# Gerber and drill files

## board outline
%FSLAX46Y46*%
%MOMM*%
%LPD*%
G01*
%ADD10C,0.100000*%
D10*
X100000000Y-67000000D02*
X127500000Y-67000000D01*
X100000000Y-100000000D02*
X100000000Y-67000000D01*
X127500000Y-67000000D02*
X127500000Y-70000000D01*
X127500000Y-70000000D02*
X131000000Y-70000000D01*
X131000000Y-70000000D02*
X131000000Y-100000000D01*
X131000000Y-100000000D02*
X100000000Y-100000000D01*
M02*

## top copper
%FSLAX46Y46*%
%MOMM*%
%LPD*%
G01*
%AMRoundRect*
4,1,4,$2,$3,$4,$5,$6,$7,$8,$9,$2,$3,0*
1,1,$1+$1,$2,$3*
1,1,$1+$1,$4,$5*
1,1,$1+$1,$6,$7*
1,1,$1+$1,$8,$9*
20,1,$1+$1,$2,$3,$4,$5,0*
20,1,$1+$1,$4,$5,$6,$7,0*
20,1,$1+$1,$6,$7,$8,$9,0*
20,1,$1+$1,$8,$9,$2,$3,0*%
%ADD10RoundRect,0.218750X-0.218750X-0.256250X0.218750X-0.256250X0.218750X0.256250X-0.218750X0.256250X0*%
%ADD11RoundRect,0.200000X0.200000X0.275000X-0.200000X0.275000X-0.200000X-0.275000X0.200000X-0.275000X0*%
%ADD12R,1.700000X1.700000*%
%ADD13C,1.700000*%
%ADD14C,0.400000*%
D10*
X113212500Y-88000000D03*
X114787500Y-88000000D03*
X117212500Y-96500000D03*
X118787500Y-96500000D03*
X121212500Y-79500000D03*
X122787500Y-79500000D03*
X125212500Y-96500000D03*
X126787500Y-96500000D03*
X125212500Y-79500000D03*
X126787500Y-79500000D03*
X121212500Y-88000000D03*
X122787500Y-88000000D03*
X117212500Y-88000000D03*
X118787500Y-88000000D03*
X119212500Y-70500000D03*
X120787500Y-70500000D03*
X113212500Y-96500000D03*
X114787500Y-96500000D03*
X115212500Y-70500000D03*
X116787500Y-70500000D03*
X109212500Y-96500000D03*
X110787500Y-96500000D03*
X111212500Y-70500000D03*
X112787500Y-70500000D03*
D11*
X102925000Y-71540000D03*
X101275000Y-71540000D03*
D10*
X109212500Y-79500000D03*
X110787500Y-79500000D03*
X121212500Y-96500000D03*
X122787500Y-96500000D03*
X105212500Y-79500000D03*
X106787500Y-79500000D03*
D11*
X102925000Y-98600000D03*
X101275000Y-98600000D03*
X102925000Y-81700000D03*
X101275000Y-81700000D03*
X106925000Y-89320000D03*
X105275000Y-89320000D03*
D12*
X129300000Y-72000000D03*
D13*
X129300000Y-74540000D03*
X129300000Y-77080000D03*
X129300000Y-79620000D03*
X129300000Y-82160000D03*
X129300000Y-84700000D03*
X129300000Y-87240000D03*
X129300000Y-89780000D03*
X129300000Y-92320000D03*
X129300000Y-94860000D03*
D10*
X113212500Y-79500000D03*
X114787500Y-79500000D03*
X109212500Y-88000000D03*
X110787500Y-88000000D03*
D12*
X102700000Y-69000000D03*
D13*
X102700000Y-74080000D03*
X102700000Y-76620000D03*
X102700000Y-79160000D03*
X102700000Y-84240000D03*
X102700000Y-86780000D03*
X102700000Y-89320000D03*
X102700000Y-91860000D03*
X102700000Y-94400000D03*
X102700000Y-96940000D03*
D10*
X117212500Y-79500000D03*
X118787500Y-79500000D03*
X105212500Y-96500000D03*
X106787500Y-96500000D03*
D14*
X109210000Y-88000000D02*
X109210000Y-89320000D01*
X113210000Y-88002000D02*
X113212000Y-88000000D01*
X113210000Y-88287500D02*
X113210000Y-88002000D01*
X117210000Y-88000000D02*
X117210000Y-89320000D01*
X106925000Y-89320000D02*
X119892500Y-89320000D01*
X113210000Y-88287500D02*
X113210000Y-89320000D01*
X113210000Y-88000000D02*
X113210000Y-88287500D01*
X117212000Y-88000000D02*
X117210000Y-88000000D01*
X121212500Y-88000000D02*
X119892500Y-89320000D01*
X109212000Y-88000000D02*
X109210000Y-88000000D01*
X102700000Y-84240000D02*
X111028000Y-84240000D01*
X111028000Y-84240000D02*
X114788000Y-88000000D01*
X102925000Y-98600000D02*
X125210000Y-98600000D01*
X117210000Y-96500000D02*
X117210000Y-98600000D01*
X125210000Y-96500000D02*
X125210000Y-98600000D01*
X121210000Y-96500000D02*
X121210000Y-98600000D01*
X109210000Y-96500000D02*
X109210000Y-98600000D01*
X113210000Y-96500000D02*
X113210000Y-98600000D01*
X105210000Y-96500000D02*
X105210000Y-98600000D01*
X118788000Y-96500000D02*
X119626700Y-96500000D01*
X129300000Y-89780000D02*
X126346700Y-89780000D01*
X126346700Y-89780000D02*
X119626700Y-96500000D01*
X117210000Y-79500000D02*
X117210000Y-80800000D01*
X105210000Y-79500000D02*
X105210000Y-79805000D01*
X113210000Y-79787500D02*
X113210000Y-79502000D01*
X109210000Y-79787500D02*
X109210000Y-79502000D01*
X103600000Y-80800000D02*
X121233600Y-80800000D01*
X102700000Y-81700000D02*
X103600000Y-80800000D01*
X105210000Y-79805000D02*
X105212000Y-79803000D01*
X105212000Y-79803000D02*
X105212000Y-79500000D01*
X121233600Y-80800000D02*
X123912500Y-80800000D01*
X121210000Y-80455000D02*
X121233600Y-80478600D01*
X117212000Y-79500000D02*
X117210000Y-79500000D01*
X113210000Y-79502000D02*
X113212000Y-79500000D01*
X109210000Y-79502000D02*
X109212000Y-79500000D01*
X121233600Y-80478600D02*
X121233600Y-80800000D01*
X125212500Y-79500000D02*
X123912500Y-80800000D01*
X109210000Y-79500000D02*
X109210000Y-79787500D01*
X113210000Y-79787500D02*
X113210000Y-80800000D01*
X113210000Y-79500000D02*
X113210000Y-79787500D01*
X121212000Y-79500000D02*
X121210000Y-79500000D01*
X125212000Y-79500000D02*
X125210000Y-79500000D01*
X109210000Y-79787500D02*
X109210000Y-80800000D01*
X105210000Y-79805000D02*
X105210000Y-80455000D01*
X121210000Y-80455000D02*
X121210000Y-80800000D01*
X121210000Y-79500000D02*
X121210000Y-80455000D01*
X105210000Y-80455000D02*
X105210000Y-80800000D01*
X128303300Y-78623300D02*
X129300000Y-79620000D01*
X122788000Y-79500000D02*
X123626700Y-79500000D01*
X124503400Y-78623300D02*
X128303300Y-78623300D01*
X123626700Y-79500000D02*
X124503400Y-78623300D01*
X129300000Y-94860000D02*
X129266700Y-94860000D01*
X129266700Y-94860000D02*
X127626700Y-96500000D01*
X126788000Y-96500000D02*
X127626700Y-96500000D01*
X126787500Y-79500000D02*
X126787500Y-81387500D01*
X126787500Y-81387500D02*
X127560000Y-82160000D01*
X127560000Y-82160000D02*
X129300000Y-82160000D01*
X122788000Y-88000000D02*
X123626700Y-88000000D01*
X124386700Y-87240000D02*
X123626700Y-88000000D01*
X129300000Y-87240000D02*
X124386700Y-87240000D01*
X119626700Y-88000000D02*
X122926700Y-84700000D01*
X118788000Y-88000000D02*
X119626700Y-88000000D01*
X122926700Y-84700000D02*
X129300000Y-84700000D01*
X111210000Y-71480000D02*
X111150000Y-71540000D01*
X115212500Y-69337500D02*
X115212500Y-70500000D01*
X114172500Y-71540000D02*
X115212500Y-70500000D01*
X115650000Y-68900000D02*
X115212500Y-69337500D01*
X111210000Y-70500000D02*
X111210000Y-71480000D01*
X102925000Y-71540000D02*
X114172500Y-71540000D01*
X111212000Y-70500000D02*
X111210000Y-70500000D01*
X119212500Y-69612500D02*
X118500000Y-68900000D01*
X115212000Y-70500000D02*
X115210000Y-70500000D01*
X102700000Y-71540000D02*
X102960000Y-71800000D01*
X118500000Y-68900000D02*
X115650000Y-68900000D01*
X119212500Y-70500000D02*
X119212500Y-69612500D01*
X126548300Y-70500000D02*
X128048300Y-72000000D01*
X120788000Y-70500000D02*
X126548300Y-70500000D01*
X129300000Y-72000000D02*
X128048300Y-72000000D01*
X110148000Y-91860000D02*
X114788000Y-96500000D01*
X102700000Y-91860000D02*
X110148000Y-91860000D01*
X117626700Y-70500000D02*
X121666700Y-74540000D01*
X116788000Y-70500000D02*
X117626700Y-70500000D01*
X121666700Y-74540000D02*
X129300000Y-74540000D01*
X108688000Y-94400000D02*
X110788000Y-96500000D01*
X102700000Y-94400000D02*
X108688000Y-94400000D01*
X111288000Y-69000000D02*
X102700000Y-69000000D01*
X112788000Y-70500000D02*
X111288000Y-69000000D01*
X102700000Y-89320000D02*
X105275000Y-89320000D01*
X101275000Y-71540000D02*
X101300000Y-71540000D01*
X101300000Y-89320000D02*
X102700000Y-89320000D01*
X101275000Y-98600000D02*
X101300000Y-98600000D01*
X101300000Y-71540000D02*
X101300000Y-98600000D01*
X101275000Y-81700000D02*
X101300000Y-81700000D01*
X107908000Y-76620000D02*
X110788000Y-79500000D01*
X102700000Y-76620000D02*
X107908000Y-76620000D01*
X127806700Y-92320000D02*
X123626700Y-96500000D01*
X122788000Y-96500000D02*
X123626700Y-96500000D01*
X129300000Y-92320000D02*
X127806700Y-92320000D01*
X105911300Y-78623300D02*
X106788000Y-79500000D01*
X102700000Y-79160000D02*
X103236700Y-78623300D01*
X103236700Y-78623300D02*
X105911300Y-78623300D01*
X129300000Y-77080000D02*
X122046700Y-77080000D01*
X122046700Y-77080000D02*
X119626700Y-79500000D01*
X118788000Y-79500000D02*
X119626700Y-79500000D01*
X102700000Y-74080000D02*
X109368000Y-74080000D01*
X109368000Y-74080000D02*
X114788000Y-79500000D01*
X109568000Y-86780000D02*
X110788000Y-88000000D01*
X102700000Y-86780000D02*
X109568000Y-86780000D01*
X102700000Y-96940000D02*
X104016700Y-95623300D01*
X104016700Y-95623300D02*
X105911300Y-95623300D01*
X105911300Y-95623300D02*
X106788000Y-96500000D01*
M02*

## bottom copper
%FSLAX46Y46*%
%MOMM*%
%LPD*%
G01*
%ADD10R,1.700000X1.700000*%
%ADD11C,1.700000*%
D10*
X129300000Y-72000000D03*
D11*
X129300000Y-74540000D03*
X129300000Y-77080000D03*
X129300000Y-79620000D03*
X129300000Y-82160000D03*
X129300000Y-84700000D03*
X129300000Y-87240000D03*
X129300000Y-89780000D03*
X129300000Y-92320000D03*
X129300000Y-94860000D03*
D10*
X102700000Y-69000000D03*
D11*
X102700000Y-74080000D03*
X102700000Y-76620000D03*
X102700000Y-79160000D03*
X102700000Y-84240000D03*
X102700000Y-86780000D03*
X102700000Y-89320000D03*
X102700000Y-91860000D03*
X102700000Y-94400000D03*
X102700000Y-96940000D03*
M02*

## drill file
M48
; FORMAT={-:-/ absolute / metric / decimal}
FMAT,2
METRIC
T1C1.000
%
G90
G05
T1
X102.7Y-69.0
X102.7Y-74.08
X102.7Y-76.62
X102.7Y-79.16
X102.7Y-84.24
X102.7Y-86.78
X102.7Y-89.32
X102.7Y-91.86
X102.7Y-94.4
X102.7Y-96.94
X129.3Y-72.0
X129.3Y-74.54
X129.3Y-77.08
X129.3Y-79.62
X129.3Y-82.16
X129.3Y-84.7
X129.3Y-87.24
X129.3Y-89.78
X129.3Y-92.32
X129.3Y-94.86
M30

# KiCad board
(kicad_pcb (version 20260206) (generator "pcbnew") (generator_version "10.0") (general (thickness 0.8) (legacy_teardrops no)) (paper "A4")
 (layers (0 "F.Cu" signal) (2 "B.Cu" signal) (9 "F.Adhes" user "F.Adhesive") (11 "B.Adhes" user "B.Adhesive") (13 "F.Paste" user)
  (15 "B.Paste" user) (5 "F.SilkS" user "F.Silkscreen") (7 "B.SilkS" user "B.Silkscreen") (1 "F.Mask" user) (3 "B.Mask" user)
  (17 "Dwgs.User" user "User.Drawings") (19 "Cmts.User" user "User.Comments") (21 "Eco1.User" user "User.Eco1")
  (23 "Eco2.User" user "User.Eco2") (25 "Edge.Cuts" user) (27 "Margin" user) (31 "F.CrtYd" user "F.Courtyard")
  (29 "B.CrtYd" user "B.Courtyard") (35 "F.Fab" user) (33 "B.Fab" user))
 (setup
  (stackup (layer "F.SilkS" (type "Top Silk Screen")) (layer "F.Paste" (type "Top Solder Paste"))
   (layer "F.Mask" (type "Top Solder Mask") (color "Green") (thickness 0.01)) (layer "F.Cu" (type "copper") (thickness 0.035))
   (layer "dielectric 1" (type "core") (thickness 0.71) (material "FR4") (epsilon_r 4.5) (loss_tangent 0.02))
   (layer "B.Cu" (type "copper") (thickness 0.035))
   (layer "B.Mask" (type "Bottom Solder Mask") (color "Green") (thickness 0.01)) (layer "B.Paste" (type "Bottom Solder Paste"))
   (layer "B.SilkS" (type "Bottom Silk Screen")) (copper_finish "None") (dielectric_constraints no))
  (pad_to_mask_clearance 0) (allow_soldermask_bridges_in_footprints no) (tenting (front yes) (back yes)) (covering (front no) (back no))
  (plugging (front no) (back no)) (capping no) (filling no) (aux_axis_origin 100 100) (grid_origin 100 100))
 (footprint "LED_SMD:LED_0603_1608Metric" (layer "F.Cu") (at 114 88)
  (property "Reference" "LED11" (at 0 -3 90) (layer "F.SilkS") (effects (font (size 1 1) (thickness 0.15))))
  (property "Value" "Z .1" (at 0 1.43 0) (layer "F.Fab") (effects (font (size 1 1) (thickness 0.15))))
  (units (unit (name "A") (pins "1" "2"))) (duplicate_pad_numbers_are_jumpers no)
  (pad "1" smd roundrect (at -0.7875 0) (size 0.875 0.95) (layers "F.Cu" "F.Mask" "F.Paste") (roundrect_rratio 0.25) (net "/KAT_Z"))
  (pad "2" smd roundrect (at 0.7875 0) (size 0.875 0.95) (layers "F.Cu" "F.Mask" "F.Paste") (roundrect_rratio 0.25) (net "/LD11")))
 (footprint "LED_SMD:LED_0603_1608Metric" (layer "F.Cu") (at 118 96.5)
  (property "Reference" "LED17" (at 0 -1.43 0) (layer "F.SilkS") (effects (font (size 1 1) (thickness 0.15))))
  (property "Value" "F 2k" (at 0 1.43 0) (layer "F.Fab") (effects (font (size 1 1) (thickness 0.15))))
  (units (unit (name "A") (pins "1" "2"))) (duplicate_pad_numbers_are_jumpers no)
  (pad "1" smd roundrect (at -0.7875 0) (size 0.875 0.95) (layers "F.Cu" "F.Mask" "F.Paste") (roundrect_rratio 0.25) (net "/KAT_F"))
  (pad "2" smd roundrect (at 0.7875 0) (size 0.875 0.95) (layers "F.Cu" "F.Mask" "F.Paste") (roundrect_rratio 0.25) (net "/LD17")))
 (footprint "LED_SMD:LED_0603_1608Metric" (layer "F.Cu") (at 122 79.5)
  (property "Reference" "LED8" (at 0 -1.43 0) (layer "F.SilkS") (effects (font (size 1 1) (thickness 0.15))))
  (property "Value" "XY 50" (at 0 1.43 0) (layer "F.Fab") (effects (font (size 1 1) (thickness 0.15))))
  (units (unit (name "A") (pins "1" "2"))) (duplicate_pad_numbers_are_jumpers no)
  (pad "1" smd roundrect (at -0.7875 0) (size 0.875 0.95) (layers "F.Cu" "F.Mask" "F.Paste") (roundrect_rratio 0.25) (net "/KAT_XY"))
  (pad "2" smd roundrect (at 0.7875 0) (size 0.875 0.95) (layers "F.Cu" "F.Mask" "F.Paste") (roundrect_rratio 0.25) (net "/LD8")))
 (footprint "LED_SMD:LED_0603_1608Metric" (layer "F.Cu") (at 126 96.5)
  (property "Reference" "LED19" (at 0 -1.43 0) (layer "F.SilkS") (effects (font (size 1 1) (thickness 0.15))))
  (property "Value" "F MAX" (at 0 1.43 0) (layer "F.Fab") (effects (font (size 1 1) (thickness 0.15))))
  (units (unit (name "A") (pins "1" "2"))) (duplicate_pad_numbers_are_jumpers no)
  (pad "1" smd roundrect (at -0.7875 0) (size 0.875 0.95) (layers "F.Cu" "F.Mask" "F.Paste") (roundrect_rratio 0.25) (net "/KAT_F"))
  (pad "2" smd roundrect (at 0.7875 0) (size 0.875 0.95) (layers "F.Cu" "F.Mask" "F.Paste") (roundrect_rratio 0.25) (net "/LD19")))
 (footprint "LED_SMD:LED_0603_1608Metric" (layer "F.Cu") (at 126 79.5)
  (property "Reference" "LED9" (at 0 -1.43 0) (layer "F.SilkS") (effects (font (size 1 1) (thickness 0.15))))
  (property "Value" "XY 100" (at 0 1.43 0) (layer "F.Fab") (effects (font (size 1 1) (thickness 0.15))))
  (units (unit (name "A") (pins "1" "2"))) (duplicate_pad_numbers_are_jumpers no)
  (pad "1" smd roundrect (at -0.7875 0) (size 0.875 0.95) (layers "F.Cu" "F.Mask" "F.Paste") (roundrect_rratio 0.25) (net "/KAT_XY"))
  (pad "2" smd roundrect (at 0.7875 0) (size 0.875 0.95) (layers "F.Cu" "F.Mask" "F.Paste") (roundrect_rratio 0.25) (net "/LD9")))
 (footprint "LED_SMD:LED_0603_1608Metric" (layer "F.Cu") (at 122 88)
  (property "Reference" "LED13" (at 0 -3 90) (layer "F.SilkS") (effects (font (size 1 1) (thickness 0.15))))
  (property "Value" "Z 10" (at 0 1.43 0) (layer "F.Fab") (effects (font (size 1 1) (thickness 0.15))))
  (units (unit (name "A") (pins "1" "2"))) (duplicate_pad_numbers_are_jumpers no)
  (pad "1" smd roundrect (at -0.7875 0) (size 0.875 0.95) (layers "F.Cu" "F.Mask" "F.Paste") (roundrect_rratio 0.25) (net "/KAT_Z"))
  (pad "2" smd roundrect (at 0.7875 0) (size 0.875 0.95) (layers "F.Cu" "F.Mask" "F.Paste") (roundrect_rratio 0.25) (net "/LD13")))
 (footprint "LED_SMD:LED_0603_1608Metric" (layer "F.Cu") (at 118 88)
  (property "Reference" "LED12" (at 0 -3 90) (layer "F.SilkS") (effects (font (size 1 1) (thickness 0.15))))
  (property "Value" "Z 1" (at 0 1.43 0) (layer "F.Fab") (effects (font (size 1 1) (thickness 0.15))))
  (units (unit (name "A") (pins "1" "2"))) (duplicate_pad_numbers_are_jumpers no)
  (pad "1" smd roundrect (at -0.7875 0) (size 0.875 0.95) (layers "F.Cu" "F.Mask" "F.Paste") (roundrect_rratio 0.25) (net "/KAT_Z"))
  (pad "2" smd roundrect (at 0.7875 0) (size 0.875 0.95) (layers "F.Cu" "F.Mask" "F.Paste") (roundrect_rratio 0.25) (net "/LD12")))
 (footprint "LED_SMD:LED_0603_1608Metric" (layer "F.Cu") (at 120 70.5)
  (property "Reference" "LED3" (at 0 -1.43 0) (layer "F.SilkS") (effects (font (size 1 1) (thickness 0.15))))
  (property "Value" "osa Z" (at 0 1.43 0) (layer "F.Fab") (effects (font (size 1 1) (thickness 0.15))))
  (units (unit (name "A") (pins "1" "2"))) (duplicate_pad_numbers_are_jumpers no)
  (pad "1" smd roundrect (at -0.7875 0) (size 0.875 0.95) (layers "F.Cu" "F.Mask" "F.Paste") (roundrect_rratio 0.25) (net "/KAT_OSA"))
  (pad "2" smd roundrect (at 0.7875 0) (size 0.875 0.95) (layers "F.Cu" "F.Mask" "F.Paste") (roundrect_rratio 0.25) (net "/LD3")))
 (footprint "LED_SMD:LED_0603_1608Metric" (layer "F.Cu") (at 114 96.5)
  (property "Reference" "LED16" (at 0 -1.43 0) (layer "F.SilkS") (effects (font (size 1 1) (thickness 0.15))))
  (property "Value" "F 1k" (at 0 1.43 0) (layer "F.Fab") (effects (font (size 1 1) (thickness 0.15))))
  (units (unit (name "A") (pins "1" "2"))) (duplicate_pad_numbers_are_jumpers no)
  (pad "1" smd roundrect (at -0.7875 0) (size 0.875 0.95) (layers "F.Cu" "F.Mask" "F.Paste") (roundrect_rratio 0.25) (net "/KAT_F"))
  (pad "2" smd roundrect (at 0.7875 0) (size 0.875 0.95) (layers "F.Cu" "F.Mask" "F.Paste") (roundrect_rratio 0.25) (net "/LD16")))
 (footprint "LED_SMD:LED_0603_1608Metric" (layer "F.Cu") (at 116 70.5)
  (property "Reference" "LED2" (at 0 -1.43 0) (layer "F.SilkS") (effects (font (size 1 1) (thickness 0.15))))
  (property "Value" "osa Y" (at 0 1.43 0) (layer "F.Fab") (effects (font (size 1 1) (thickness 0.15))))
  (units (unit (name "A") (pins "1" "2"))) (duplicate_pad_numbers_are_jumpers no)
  (pad "1" smd roundrect (at -0.7875 0) (size 0.875 0.95) (layers "F.Cu" "F.Mask" "F.Paste") (roundrect_rratio 0.25) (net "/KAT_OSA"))
  (pad "2" smd roundrect (at 0.7875 0) (size 0.875 0.95) (layers "F.Cu" "F.Mask" "F.Paste") (roundrect_rratio 0.25) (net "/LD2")))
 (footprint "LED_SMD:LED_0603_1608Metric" (layer "F.Cu") (at 110 96.5)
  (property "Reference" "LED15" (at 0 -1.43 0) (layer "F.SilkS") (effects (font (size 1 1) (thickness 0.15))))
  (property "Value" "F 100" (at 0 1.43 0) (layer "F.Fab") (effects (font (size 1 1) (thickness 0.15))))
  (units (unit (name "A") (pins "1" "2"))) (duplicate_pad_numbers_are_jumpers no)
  (pad "1" smd roundrect (at -0.7875 0) (size 0.875 0.95) (layers "F.Cu" "F.Mask" "F.Paste") (roundrect_rratio 0.25) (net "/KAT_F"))
  (pad "2" smd roundrect (at 0.7875 0) (size 0.875 0.95) (layers "F.Cu" "F.Mask" "F.Paste") (roundrect_rratio 0.25) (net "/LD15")))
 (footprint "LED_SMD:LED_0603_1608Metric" (layer "F.Cu") (at 112 70.5)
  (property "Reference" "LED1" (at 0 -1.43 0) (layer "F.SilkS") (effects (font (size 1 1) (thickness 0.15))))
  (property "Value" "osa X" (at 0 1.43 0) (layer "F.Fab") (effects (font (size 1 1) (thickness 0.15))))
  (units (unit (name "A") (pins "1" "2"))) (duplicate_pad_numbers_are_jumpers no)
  (pad "1" smd roundrect (at -0.7875 0) (size 0.875 0.95) (layers "F.Cu" "F.Mask" "F.Paste") (roundrect_rratio 0.25) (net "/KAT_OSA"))
  (pad "2" smd roundrect (at 0.7875 0) (size 0.875 0.95) (layers "F.Cu" "F.Mask" "F.Paste") (roundrect_rratio 0.25) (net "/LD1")))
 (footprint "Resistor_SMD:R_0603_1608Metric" (layer "F.Cu") (at 102.1 71.54 180)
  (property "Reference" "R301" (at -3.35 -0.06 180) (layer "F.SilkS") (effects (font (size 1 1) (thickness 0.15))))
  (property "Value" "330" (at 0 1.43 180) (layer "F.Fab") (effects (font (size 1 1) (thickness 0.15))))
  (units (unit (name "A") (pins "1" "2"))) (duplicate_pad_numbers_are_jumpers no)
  (pad "1" smd roundrect (at -0.825 0 180) (size 0.8 0.95) (layers "F.Cu" "F.Mask" "F.Paste") (roundrect_rratio 0.25) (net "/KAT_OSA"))
  (pad "2" smd roundrect (at 0.825 0 180) (size 0.8 0.95) (layers "F.Cu" "F.Mask" "F.Paste") (roundrect_rratio 0.25) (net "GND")))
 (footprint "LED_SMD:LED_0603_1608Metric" (layer "F.Cu") (at 110 79.5)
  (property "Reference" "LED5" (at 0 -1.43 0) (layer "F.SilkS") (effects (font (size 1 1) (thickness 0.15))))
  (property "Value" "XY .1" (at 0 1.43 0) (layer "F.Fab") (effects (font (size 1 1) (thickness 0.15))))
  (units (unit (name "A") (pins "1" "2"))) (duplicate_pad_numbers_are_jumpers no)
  (pad "1" smd roundrect (at -0.7875 0) (size 0.875 0.95) (layers "F.Cu" "F.Mask" "F.Paste") (roundrect_rratio 0.25) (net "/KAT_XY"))
  (pad "2" smd roundrect (at 0.7875 0) (size 0.875 0.95) (layers "F.Cu" "F.Mask" "F.Paste") (roundrect_rratio 0.25) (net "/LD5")))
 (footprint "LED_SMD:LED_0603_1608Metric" (layer "F.Cu") (at 122 96.5)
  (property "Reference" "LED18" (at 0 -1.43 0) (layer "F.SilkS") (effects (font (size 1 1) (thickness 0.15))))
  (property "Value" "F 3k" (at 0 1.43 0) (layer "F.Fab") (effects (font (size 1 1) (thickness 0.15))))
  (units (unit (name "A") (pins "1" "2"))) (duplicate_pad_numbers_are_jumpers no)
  (pad "1" smd roundrect (at -0.7875 0) (size 0.875 0.95) (layers "F.Cu" "F.Mask" "F.Paste") (roundrect_rratio 0.25) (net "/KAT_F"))
  (pad "2" smd roundrect (at 0.7875 0) (size 0.875 0.95) (layers "F.Cu" "F.Mask" "F.Paste") (roundrect_rratio 0.25) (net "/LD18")))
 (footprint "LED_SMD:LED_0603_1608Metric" (layer "F.Cu") (at 106 79.5)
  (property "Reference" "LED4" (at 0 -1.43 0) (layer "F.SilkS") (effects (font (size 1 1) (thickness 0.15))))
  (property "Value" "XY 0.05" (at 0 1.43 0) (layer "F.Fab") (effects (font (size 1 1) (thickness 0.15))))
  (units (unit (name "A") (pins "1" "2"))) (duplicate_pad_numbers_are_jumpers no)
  (pad "1" smd roundrect (at -0.7875 0) (size 0.875 0.95) (layers "F.Cu" "F.Mask" "F.Paste") (roundrect_rratio 0.25) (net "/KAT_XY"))
  (pad "2" smd roundrect (at 0.7875 0) (size 0.875 0.95) (layers "F.Cu" "F.Mask" "F.Paste") (roundrect_rratio 0.25) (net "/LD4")))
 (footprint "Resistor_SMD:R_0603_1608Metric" (layer "F.Cu") (at 102.1 98.6 180)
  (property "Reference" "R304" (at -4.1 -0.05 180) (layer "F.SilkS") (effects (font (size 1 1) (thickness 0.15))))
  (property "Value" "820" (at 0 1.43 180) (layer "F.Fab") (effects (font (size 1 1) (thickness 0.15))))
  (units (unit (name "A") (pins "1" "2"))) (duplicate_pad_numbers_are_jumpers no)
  (pad "1" smd roundrect (at -0.825 0 180) (size 0.8 0.95) (layers "F.Cu" "F.Mask" "F.Paste") (roundrect_rratio 0.25) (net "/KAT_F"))
  (pad "2" smd roundrect (at 0.825 0 180) (size 0.8 0.95) (layers "F.Cu" "F.Mask" "F.Paste") (roundrect_rratio 0.25) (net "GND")))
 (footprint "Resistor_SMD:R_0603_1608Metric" (layer "F.Cu") (at 102.1 81.7 180)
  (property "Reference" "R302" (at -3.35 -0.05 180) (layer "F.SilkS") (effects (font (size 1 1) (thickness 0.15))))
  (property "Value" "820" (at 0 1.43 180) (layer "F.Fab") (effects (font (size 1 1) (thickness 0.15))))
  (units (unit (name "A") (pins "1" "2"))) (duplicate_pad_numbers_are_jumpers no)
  (pad "1" smd roundrect (at -0.825 0 180) (size 0.8 0.95) (layers "F.Cu" "F.Mask" "F.Paste") (roundrect_rratio 0.25) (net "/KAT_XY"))
  (pad "2" smd roundrect (at 0.825 0 180) (size 0.8 0.95) (layers "F.Cu" "F.Mask" "F.Paste") (roundrect_rratio 0.25) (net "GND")))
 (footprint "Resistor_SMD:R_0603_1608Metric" (layer "F.Cu") (at 106.1 89.32 180)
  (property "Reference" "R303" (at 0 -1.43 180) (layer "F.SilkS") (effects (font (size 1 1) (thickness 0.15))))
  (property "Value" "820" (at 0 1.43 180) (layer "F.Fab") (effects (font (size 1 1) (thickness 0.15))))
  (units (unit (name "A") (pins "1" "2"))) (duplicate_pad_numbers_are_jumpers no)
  (pad "1" smd roundrect (at -0.825 0 180) (size 0.8 0.95) (layers "F.Cu" "F.Mask" "F.Paste") (roundrect_rratio 0.25) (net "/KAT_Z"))
  (pad "2" smd roundrect (at 0.825 0 180) (size 0.8 0.95) (layers "F.Cu" "F.Mask" "F.Paste") (roundrect_rratio 0.25) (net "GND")))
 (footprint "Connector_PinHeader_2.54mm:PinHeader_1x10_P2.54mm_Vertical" (layer "F.Cu") (at 129.3 72)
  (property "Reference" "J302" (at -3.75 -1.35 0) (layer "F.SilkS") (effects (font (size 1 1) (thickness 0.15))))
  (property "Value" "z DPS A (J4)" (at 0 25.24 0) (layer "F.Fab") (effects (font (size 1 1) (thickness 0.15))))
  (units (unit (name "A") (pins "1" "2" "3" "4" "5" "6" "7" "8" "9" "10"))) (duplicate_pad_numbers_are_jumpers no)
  (pad "1" thru_hole rect (at 0 0) (size 1.7 1.7) (drill 1) (layers "*.Cu" "*.Mask") (remove_unused_layers no) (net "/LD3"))
  (pad "2" thru_hole circle (at 0 2.54) (size 1.7 1.7) (drill 1) (layers "*.Cu" "*.Mask") (remove_unused_layers no) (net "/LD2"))
  (pad "3" thru_hole circle (at 0 5.08) (size 1.7 1.7) (drill 1) (layers "*.Cu" "*.Mask") (remove_unused_layers no) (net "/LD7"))
  (pad "4" thru_hole circle (at 0 7.62) (size 1.7 1.7) (drill 1) (layers "*.Cu" "*.Mask") (remove_unused_layers no) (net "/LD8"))
  (pad "5" thru_hole circle (at 0 10.16) (size 1.7 1.7) (drill 1) (layers "*.Cu" "*.Mask") (remove_unused_layers no) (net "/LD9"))
  (pad "6" thru_hole circle (at 0 12.7) (size 1.7 1.7) (drill 1) (layers "*.Cu" "*.Mask") (remove_unused_layers no) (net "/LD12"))
  (pad "7" thru_hole circle (at 0 15.24) (size 1.7 1.7) (drill 1) (layers "*.Cu" "*.Mask") (remove_unused_layers no) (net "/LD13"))
  (pad "8" thru_hole circle (at 0 17.78) (size 1.7 1.7) (drill 1) (layers "*.Cu" "*.Mask") (remove_unused_layers no) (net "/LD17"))
  (pad "9" thru_hole circle (at 0 20.32) (size 1.7 1.7) (drill 1) (layers "*.Cu" "*.Mask") (remove_unused_layers no) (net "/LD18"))
  (pad "10" thru_hole circle (at 0 22.86) (size 1.7 1.7) (drill 1) (layers "*.Cu" "*.Mask") (remove_unused_layers no) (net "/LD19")))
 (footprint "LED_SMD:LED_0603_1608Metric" (layer "F.Cu") (at 114 79.5)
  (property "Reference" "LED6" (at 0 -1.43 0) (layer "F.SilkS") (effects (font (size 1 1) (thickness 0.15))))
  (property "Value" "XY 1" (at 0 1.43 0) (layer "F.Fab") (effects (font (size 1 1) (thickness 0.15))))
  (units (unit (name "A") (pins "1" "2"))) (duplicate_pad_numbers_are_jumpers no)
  (pad "1" smd roundrect (at -0.7875 0) (size 0.875 0.95) (layers "F.Cu" "F.Mask" "F.Paste") (roundrect_rratio 0.25) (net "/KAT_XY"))
  (pad "2" smd roundrect (at 0.7875 0) (size 0.875 0.95) (layers "F.Cu" "F.Mask" "F.Paste") (roundrect_rratio 0.25) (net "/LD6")))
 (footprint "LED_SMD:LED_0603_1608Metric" (layer "F.Cu") (at 110 88)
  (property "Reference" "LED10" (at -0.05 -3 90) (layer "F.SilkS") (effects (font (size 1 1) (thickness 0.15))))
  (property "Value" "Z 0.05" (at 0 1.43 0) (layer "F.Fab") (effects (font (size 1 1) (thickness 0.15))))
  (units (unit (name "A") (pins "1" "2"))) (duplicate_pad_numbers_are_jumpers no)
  (pad "1" smd roundrect (at -0.7875 0) (size 0.875 0.95) (layers "F.Cu" "F.Mask" "F.Paste") (roundrect_rratio 0.25) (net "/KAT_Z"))
  (pad "2" smd roundrect (at 0.7875 0) (size 0.875 0.95) (layers "F.Cu" "F.Mask" "F.Paste") (roundrect_rratio 0.25) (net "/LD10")))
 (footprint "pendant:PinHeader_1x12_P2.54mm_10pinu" (layer "F.Cu") (at 102.7 69)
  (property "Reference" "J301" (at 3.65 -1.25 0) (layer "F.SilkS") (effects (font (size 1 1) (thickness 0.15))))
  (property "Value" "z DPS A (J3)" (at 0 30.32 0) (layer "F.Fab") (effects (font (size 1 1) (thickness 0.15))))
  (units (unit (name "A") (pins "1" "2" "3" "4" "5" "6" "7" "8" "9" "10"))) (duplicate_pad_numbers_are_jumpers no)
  (pad "1" thru_hole rect (at 0 0) (size 1.7 1.7) (drill 1) (layers "*.Cu" "*.Mask") (remove_unused_layers no) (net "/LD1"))
  (pad "2" thru_hole circle (at 0 5.08) (size 1.7 1.7) (drill 1) (layers "*.Cu" "*.Mask") (remove_unused_layers no) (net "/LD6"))
  (pad "3" thru_hole circle (at 0 7.62) (size 1.7 1.7) (drill 1) (layers "*.Cu" "*.Mask") (remove_unused_layers no) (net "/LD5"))
  (pad "4" thru_hole circle (at 0 10.16) (size 1.7 1.7) (drill 1) (layers "*.Cu" "*.Mask") (remove_unused_layers no) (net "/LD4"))
  (pad "5" thru_hole circle (at 0 15.24) (size 1.7 1.7) (drill 1) (layers "*.Cu" "*.Mask") (remove_unused_layers no) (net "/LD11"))
  (pad "6" thru_hole circle (at 0 17.78) (size 1.7 1.7) (drill 1) (layers "*.Cu" "*.Mask") (remove_unused_layers no) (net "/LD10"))
  (pad "7" thru_hole circle (at 0 20.32) (size 1.7 1.7) (drill 1) (layers "*.Cu" "*.Mask") (remove_unused_layers no) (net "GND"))
  (pad "8" thru_hole circle (at 0 22.86) (size 1.7 1.7) (drill 1) (layers "*.Cu" "*.Mask") (remove_unused_layers no) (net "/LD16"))
  (pad "9" thru_hole circle (at 0 25.4) (size 1.7 1.7) (drill 1) (layers "*.Cu" "*.Mask") (remove_unused_layers no) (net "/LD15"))
  (pad "10" thru_hole circle (at 0 27.94) (size 1.7 1.7) (drill 1) (layers "*.Cu" "*.Mask") (remove_unused_layers no) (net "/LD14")))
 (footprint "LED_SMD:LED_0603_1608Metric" (layer "F.Cu") (at 118 79.5)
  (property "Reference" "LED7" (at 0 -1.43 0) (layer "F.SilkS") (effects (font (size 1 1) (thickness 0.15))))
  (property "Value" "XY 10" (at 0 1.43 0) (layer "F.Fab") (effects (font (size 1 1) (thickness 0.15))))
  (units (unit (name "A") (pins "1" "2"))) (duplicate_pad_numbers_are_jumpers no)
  (pad "1" smd roundrect (at -0.7875 0) (size 0.875 0.95) (layers "F.Cu" "F.Mask" "F.Paste") (roundrect_rratio 0.25) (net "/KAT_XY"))
  (pad "2" smd roundrect (at 0.7875 0) (size 0.875 0.95) (layers "F.Cu" "F.Mask" "F.Paste") (roundrect_rratio 0.25) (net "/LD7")))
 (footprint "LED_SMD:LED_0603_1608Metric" (layer "F.Cu") (at 106 96.5)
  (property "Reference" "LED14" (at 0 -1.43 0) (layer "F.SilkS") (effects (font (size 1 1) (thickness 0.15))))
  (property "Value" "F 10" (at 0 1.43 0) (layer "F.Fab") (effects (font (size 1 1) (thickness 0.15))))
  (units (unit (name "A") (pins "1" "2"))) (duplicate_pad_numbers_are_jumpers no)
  (pad "1" smd roundrect (at -0.7875 0) (size 0.875 0.95) (layers "F.Cu" "F.Mask" "F.Paste") (roundrect_rratio 0.25) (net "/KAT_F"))
  (pad "2" smd roundrect (at 0.7875 0) (size 0.875 0.95) (layers "F.Cu" "F.Mask" "F.Paste") (roundrect_rratio 0.25) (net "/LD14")))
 (gr_line (start 100 67) (end 127.5 67) (stroke (width 0.1) (type default)) (layer "Edge.Cuts"))
 (gr_line (start 100 100) (end 100 67) (stroke (width 0.1) (type default)) (layer "Edge.Cuts"))
 (gr_line (start 127.5 67) (end 127.5 70) (stroke (width 0.1) (type default)) (layer "Edge.Cuts"))
 (gr_line (start 127.5 70) (end 131 70) (stroke (width 0.1) (type default)) (layer "Edge.Cuts"))
 (gr_line (start 131 70) (end 131 100) (stroke (width 0.1) (type default)) (layer "Edge.Cuts"))
 (gr_line (start 131 100) (end 100 100) (stroke (width 0.1) (type default)) (layer "Edge.Cuts"))
 (segment (start 109.21 88) (end 109.21 89.32) (width 0.4) (layer "F.Cu") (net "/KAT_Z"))
 (segment (start 113.21 88.002) (end 113.212 88) (width 0.4) (layer "F.Cu") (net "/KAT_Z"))
 (segment (start 113.21 88.2875) (end 113.21 88.002) (width 0.4) (layer "F.Cu") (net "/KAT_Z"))
 (segment (start 117.21 88) (end 117.21 89.32) (width 0.4) (layer "F.Cu") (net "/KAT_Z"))
 (segment (start 106.925 89.32) (end 119.8925 89.32) (width 0.4) (layer "F.Cu") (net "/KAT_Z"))
 (segment (start 113.21 88.2875) (end 113.21 89.32) (width 0.4) (layer "F.Cu") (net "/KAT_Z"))
 (segment (start 113.21 88) (end 113.21 88.2875) (width 0.4) (layer "F.Cu") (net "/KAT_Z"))
 (segment (start 117.212 88) (end 117.21 88) (width 0.4) (layer "F.Cu") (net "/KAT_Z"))
 (segment (start 121.2125 88) (end 119.8925 89.32) (width 0.4) (layer "F.Cu") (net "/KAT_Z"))
 (segment (start 109.212 88) (end 109.21 88) (width 0.4) (layer "F.Cu") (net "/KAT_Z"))
 (segment (start 102.7 84.24) (end 111.028 84.24) (width 0.4) (layer "F.Cu") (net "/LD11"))
 (segment (start 111.028 84.24) (end 114.788 88) (width 0.4) (layer "F.Cu") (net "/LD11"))
 (segment (start 102.925 98.6) (end 125.21 98.6) (width 0.4) (layer "F.Cu") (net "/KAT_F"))
 (segment (start 117.21 96.5) (end 117.21 98.6) (width 0.4) (layer "F.Cu") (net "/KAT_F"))
 (segment (start 125.21 96.5) (end 125.21 98.6) (width 0.4) (layer "F.Cu") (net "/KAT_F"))
 (segment (start 121.21 96.5) (end 121.21 98.6) (width 0.4) (layer "F.Cu") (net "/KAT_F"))
 (segment (start 109.21 96.5) (end 109.21 98.6) (width 0.4) (layer "F.Cu") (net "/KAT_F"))
 (segment (start 113.21 96.5) (end 113.21 98.6) (width 0.4) (layer "F.Cu") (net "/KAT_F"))
 (segment (start 105.21 96.5) (end 105.21 98.6) (width 0.4) (layer "F.Cu") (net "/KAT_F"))
 (segment (start 118.788 96.5) (end 119.6267 96.5) (width 0.4) (layer "F.Cu") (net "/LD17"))
 (segment (start 129.3 89.78) (end 126.3467 89.78) (width 0.4) (layer "F.Cu") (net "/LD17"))
 (segment (start 126.3467 89.78) (end 119.6267 96.5) (width 0.4) (layer "F.Cu") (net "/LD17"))
 (segment (start 117.21 79.5) (end 117.21 80.8) (width 0.4) (layer "F.Cu") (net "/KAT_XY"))
 (segment (start 105.21 79.5) (end 105.21 79.805) (width 0.4) (layer "F.Cu") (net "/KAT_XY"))
 (segment (start 113.21 79.7875) (end 113.21 79.502) (width 0.4) (layer "F.Cu") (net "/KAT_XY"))
 (segment (start 109.21 79.7875) (end 109.21 79.502) (width 0.4) (layer "F.Cu") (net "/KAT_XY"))
 (segment (start 103.6 80.8) (end 121.2336 80.8) (width 0.4) (layer "F.Cu") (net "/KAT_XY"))
 (segment (start 102.7 81.7) (end 103.6 80.8) (width 0.4) (layer "F.Cu") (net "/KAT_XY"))
 (segment (start 105.21 79.805) (end 105.212 79.803) (width 0.4) (layer "F.Cu") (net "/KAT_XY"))
 (segment (start 105.212 79.803) (end 105.212 79.5) (width 0.4) (layer "F.Cu") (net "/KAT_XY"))
 (segment (start 121.2336 80.8) (end 123.9125 80.8) (width 0.4) (layer "F.Cu") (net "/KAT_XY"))
 (segment (start 121.21 80.455) (end 121.2336 80.4786) (width 0.4) (layer "F.Cu") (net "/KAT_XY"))
 (segment (start 117.212 79.5) (end 117.21 79.5) (width 0.4) (layer "F.Cu") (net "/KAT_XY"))
 (segment (start 113.21 79.502) (end 113.212 79.5) (width 0.4) (layer "F.Cu") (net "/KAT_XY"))
 (segment (start 109.21 79.502) (end 109.212 79.5) (width 0.4) (layer "F.Cu") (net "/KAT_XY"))
 (segment (start 121.2336 80.4786) (end 121.2336 80.8) (width 0.4) (layer "F.Cu") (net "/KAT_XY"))
 (segment (start 125.2125 79.5) (end 123.9125 80.8) (width 0.4) (layer "F.Cu") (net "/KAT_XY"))
 (segment (start 109.21 79.5) (end 109.21 79.7875) (width 0.4) (layer "F.Cu") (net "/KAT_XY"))
 (segment (start 113.21 79.7875) (end 113.21 80.8) (width 0.4) (layer "F.Cu") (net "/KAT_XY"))
 (segment (start 113.21 79.5) (end 113.21 79.7875) (width 0.4) (layer "F.Cu") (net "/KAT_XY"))
 (segment (start 121.212 79.5) (end 121.21 79.5) (width 0.4) (layer "F.Cu") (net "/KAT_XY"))
 (segment (start 125.212 79.5) (end 125.21 79.5) (width 0.4) (layer "F.Cu") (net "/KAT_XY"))
 (segment (start 109.21 79.7875) (end 109.21 80.8) (width 0.4) (layer "F.Cu") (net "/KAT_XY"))
 (segment (start 105.21 79.805) (end 105.21 80.455) (width 0.4) (layer "F.Cu") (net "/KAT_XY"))
 (segment (start 121.21 80.455) (end 121.21 80.8) (width 0.4) (layer "F.Cu") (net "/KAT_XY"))
 (segment (start 121.21 79.5) (end 121.21 80.455) (width 0.4) (layer "F.Cu") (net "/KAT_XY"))
 (segment (start 105.21 80.455) (end 105.21 80.8) (width 0.4) (layer "F.Cu") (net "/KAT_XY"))
 (segment (start 128.3033 78.6233) (end 129.3 79.62) (width 0.4) (layer "F.Cu") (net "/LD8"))
 (segment (start 122.788 79.5) (end 123.6267 79.5) (width 0.4) (layer "F.Cu") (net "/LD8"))
 (segment (start 124.5034 78.6233) (end 128.3033 78.6233) (width 0.4) (layer "F.Cu") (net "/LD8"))
 (segment (start 123.6267 79.5) (end 124.5034 78.6233) (width 0.4) (layer "F.Cu") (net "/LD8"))
 (segment (start 129.3 94.86) (end 129.2667 94.86) (width 0.4) (layer "F.Cu") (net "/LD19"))
 (segment (start 129.2667 94.86) (end 127.6267 96.5) (width 0.4) (layer "F.Cu") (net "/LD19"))
 (segment (start 126.788 96.5) (end 127.6267 96.5) (width 0.4) (layer "F.Cu") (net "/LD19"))
 (segment (start 126.7875 79.5) (end 126.7875 81.3875) (width 0.4) (layer "F.Cu") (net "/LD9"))
 (segment (start 126.7875 81.3875) (end 127.56 82.16) (width 0.4) (layer "F.Cu") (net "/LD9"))
 (segment (start 127.56 82.16) (end 129.3 82.16) (width 0.4) (layer "F.Cu") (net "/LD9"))
 (segment (start 122.788 88) (end 123.6267 88) (width 0.4) (layer "F.Cu") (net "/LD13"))
 (segment (start 124.3867 87.24) (end 123.6267 88) (width 0.4) (layer "F.Cu") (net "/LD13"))
 (segment (start 129.3 87.24) (end 124.3867 87.24) (width 0.4) (layer "F.Cu") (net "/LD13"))
 (segment (start 119.6267 88) (end 122.9267 84.7) (width 0.4) (layer "F.Cu") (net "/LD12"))
 (segment (start 118.788 88) (end 119.6267 88) (width 0.4) (layer "F.Cu") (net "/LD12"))
 (segment (start 122.9267 84.7) (end 129.3 84.7) (width 0.4) (layer "F.Cu") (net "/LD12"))
 (segment (start 111.21 71.48) (end 111.15 71.54) (width 0.4) (layer "F.Cu") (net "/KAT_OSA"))
 (segment (start 115.2125 69.3375) (end 115.2125 70.5) (width 0.4) (layer "F.Cu") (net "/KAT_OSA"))
 (segment (start 114.1725 71.54) (end 115.2125 70.5) (width 0.4) (layer "F.Cu") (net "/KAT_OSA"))
 (segment (start 115.65 68.9) (end 115.2125 69.3375) (width 0.4) (layer "F.Cu") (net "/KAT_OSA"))
 (segment (start 111.21 70.5) (end 111.21 71.48) (width 0.4) (layer "F.Cu") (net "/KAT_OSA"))
 (segment (start 102.925 71.54) (end 114.1725 71.54) (width 0.4) (layer "F.Cu") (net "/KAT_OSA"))
 (segment (start 111.212 70.5) (end 111.21 70.5) (width 0.4) (layer "F.Cu") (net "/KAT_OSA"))
 (segment (start 119.2125 69.6125) (end 118.5 68.9) (width 0.4) (layer "F.Cu") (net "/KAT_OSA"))
 (segment (start 115.212 70.5) (end 115.21 70.5) (width 0.4) (layer "F.Cu") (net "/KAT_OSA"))
 (segment (start 102.7 71.54) (end 102.96 71.8) (width 0.4) (layer "F.Cu") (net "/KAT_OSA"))
 (segment (start 118.5 68.9) (end 115.65 68.9) (width 0.4) (layer "F.Cu") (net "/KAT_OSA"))
 (segment (start 119.2125 70.5) (end 119.2125 69.6125) (width 0.4) (layer "F.Cu") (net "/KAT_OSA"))
 (segment (start 126.5483 70.5) (end 128.0483 72) (width 0.4) (layer "F.Cu") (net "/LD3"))
 (segment (start 120.788 70.5) (end 126.5483 70.5) (width 0.4) (layer "F.Cu") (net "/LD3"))
 (segment (start 129.3 72) (end 128.0483 72) (width 0.4) (layer "F.Cu") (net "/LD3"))
 (segment (start 110.148 91.86) (end 114.788 96.5) (width 0.4) (layer "F.Cu") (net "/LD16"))
 (segment (start 102.7 91.86) (end 110.148 91.86) (width 0.4) (layer "F.Cu") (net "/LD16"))
 (segment (start 117.6267 70.5) (end 121.6667 74.54) (width 0.4) (layer "F.Cu") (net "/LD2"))
 (segment (start 116.788 70.5) (end 117.6267 70.5) (width 0.4) (layer "F.Cu") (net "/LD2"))
 (segment (start 121.6667 74.54) (end 129.3 74.54) (width 0.4) (layer "F.Cu") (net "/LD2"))
 (segment (start 108.688 94.4) (end 110.788 96.5) (width 0.4) (layer "F.Cu") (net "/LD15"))
 (segment (start 102.7 94.4) (end 108.688 94.4) (width 0.4) (layer "F.Cu") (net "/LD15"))
 (segment (start 111.288 69) (end 102.7 69) (width 0.4) (layer "F.Cu") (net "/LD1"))
 (segment (start 112.788 70.5) (end 111.288 69) (width 0.4) (layer "F.Cu") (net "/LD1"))
 (segment (start 102.7 89.32) (end 105.275 89.32) (width 0.4) (layer "F.Cu") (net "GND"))
 (segment (start 101.275 71.54) (end 101.3 71.54) (width 0.4) (layer "F.Cu") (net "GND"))
 (segment (start 101.3 89.32) (end 102.7 89.32) (width 0.4) (layer "F.Cu") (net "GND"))
 (segment (start 101.275 98.6) (end 101.3 98.6) (width 0.4) (layer "F.Cu") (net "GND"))
 (segment (start 101.3 71.54) (end 101.3 98.6) (width 0.4) (layer "F.Cu") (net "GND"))
 (segment (start 101.275 81.7) (end 101.3 81.7) (width 0.4) (layer "F.Cu") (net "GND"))
 (segment (start 107.908 76.62) (end 110.788 79.5) (width 0.4) (layer "F.Cu") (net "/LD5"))
 (segment (start 102.7 76.62) (end 107.908 76.62) (width 0.4) (layer "F.Cu") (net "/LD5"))
 (segment (start 127.8067 92.32) (end 123.6267 96.5) (width 0.4) (layer "F.Cu") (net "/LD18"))
 (segment (start 122.788 96.5) (end 123.6267 96.5) (width 0.4) (layer "F.Cu") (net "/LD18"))
 (segment (start 129.3 92.32) (end 127.8067 92.32) (width 0.4) (layer "F.Cu") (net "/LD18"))
 (segment (start 105.9113 78.6233) (end 106.788 79.5) (width 0.4) (layer "F.Cu") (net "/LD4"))
 (segment (start 102.7 79.16) (end 103.2367 78.6233) (width 0.4) (layer "F.Cu") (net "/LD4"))
 (segment (start 103.2367 78.6233) (end 105.9113 78.6233) (width 0.4) (layer "F.Cu") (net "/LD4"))
 (segment (start 129.3 77.08) (end 122.0467 77.08) (width 0.4) (layer "F.Cu") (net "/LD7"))
 (segment (start 122.0467 77.08) (end 119.6267 79.5) (width 0.4) (layer "F.Cu") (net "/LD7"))
 (segment (start 118.788 79.5) (end 119.6267 79.5) (width 0.4) (layer "F.Cu") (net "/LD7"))
 (segment (start 102.7 74.08) (end 109.368 74.08) (width 0.4) (layer "F.Cu") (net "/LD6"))
 (segment (start 109.368 74.08) (end 114.788 79.5) (width 0.4) (layer "F.Cu") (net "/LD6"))
 (segment (start 109.568 86.78) (end 110.788 88) (width 0.4) (layer "F.Cu") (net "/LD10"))
 (segment (start 102.7 86.78) (end 109.568 86.78) (width 0.4) (layer "F.Cu") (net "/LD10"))
 (segment (start 102.7 96.94) (end 104.0167 95.6233) (width 0.4) (layer "F.Cu") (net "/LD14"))
 (segment (start 104.0167 95.6233) (end 105.9113 95.6233) (width 0.4) (layer "F.Cu") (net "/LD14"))
 (segment (start 105.9113 95.6233) (end 106.788 96.5) (width 0.4) (layer "F.Cu") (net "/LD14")))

